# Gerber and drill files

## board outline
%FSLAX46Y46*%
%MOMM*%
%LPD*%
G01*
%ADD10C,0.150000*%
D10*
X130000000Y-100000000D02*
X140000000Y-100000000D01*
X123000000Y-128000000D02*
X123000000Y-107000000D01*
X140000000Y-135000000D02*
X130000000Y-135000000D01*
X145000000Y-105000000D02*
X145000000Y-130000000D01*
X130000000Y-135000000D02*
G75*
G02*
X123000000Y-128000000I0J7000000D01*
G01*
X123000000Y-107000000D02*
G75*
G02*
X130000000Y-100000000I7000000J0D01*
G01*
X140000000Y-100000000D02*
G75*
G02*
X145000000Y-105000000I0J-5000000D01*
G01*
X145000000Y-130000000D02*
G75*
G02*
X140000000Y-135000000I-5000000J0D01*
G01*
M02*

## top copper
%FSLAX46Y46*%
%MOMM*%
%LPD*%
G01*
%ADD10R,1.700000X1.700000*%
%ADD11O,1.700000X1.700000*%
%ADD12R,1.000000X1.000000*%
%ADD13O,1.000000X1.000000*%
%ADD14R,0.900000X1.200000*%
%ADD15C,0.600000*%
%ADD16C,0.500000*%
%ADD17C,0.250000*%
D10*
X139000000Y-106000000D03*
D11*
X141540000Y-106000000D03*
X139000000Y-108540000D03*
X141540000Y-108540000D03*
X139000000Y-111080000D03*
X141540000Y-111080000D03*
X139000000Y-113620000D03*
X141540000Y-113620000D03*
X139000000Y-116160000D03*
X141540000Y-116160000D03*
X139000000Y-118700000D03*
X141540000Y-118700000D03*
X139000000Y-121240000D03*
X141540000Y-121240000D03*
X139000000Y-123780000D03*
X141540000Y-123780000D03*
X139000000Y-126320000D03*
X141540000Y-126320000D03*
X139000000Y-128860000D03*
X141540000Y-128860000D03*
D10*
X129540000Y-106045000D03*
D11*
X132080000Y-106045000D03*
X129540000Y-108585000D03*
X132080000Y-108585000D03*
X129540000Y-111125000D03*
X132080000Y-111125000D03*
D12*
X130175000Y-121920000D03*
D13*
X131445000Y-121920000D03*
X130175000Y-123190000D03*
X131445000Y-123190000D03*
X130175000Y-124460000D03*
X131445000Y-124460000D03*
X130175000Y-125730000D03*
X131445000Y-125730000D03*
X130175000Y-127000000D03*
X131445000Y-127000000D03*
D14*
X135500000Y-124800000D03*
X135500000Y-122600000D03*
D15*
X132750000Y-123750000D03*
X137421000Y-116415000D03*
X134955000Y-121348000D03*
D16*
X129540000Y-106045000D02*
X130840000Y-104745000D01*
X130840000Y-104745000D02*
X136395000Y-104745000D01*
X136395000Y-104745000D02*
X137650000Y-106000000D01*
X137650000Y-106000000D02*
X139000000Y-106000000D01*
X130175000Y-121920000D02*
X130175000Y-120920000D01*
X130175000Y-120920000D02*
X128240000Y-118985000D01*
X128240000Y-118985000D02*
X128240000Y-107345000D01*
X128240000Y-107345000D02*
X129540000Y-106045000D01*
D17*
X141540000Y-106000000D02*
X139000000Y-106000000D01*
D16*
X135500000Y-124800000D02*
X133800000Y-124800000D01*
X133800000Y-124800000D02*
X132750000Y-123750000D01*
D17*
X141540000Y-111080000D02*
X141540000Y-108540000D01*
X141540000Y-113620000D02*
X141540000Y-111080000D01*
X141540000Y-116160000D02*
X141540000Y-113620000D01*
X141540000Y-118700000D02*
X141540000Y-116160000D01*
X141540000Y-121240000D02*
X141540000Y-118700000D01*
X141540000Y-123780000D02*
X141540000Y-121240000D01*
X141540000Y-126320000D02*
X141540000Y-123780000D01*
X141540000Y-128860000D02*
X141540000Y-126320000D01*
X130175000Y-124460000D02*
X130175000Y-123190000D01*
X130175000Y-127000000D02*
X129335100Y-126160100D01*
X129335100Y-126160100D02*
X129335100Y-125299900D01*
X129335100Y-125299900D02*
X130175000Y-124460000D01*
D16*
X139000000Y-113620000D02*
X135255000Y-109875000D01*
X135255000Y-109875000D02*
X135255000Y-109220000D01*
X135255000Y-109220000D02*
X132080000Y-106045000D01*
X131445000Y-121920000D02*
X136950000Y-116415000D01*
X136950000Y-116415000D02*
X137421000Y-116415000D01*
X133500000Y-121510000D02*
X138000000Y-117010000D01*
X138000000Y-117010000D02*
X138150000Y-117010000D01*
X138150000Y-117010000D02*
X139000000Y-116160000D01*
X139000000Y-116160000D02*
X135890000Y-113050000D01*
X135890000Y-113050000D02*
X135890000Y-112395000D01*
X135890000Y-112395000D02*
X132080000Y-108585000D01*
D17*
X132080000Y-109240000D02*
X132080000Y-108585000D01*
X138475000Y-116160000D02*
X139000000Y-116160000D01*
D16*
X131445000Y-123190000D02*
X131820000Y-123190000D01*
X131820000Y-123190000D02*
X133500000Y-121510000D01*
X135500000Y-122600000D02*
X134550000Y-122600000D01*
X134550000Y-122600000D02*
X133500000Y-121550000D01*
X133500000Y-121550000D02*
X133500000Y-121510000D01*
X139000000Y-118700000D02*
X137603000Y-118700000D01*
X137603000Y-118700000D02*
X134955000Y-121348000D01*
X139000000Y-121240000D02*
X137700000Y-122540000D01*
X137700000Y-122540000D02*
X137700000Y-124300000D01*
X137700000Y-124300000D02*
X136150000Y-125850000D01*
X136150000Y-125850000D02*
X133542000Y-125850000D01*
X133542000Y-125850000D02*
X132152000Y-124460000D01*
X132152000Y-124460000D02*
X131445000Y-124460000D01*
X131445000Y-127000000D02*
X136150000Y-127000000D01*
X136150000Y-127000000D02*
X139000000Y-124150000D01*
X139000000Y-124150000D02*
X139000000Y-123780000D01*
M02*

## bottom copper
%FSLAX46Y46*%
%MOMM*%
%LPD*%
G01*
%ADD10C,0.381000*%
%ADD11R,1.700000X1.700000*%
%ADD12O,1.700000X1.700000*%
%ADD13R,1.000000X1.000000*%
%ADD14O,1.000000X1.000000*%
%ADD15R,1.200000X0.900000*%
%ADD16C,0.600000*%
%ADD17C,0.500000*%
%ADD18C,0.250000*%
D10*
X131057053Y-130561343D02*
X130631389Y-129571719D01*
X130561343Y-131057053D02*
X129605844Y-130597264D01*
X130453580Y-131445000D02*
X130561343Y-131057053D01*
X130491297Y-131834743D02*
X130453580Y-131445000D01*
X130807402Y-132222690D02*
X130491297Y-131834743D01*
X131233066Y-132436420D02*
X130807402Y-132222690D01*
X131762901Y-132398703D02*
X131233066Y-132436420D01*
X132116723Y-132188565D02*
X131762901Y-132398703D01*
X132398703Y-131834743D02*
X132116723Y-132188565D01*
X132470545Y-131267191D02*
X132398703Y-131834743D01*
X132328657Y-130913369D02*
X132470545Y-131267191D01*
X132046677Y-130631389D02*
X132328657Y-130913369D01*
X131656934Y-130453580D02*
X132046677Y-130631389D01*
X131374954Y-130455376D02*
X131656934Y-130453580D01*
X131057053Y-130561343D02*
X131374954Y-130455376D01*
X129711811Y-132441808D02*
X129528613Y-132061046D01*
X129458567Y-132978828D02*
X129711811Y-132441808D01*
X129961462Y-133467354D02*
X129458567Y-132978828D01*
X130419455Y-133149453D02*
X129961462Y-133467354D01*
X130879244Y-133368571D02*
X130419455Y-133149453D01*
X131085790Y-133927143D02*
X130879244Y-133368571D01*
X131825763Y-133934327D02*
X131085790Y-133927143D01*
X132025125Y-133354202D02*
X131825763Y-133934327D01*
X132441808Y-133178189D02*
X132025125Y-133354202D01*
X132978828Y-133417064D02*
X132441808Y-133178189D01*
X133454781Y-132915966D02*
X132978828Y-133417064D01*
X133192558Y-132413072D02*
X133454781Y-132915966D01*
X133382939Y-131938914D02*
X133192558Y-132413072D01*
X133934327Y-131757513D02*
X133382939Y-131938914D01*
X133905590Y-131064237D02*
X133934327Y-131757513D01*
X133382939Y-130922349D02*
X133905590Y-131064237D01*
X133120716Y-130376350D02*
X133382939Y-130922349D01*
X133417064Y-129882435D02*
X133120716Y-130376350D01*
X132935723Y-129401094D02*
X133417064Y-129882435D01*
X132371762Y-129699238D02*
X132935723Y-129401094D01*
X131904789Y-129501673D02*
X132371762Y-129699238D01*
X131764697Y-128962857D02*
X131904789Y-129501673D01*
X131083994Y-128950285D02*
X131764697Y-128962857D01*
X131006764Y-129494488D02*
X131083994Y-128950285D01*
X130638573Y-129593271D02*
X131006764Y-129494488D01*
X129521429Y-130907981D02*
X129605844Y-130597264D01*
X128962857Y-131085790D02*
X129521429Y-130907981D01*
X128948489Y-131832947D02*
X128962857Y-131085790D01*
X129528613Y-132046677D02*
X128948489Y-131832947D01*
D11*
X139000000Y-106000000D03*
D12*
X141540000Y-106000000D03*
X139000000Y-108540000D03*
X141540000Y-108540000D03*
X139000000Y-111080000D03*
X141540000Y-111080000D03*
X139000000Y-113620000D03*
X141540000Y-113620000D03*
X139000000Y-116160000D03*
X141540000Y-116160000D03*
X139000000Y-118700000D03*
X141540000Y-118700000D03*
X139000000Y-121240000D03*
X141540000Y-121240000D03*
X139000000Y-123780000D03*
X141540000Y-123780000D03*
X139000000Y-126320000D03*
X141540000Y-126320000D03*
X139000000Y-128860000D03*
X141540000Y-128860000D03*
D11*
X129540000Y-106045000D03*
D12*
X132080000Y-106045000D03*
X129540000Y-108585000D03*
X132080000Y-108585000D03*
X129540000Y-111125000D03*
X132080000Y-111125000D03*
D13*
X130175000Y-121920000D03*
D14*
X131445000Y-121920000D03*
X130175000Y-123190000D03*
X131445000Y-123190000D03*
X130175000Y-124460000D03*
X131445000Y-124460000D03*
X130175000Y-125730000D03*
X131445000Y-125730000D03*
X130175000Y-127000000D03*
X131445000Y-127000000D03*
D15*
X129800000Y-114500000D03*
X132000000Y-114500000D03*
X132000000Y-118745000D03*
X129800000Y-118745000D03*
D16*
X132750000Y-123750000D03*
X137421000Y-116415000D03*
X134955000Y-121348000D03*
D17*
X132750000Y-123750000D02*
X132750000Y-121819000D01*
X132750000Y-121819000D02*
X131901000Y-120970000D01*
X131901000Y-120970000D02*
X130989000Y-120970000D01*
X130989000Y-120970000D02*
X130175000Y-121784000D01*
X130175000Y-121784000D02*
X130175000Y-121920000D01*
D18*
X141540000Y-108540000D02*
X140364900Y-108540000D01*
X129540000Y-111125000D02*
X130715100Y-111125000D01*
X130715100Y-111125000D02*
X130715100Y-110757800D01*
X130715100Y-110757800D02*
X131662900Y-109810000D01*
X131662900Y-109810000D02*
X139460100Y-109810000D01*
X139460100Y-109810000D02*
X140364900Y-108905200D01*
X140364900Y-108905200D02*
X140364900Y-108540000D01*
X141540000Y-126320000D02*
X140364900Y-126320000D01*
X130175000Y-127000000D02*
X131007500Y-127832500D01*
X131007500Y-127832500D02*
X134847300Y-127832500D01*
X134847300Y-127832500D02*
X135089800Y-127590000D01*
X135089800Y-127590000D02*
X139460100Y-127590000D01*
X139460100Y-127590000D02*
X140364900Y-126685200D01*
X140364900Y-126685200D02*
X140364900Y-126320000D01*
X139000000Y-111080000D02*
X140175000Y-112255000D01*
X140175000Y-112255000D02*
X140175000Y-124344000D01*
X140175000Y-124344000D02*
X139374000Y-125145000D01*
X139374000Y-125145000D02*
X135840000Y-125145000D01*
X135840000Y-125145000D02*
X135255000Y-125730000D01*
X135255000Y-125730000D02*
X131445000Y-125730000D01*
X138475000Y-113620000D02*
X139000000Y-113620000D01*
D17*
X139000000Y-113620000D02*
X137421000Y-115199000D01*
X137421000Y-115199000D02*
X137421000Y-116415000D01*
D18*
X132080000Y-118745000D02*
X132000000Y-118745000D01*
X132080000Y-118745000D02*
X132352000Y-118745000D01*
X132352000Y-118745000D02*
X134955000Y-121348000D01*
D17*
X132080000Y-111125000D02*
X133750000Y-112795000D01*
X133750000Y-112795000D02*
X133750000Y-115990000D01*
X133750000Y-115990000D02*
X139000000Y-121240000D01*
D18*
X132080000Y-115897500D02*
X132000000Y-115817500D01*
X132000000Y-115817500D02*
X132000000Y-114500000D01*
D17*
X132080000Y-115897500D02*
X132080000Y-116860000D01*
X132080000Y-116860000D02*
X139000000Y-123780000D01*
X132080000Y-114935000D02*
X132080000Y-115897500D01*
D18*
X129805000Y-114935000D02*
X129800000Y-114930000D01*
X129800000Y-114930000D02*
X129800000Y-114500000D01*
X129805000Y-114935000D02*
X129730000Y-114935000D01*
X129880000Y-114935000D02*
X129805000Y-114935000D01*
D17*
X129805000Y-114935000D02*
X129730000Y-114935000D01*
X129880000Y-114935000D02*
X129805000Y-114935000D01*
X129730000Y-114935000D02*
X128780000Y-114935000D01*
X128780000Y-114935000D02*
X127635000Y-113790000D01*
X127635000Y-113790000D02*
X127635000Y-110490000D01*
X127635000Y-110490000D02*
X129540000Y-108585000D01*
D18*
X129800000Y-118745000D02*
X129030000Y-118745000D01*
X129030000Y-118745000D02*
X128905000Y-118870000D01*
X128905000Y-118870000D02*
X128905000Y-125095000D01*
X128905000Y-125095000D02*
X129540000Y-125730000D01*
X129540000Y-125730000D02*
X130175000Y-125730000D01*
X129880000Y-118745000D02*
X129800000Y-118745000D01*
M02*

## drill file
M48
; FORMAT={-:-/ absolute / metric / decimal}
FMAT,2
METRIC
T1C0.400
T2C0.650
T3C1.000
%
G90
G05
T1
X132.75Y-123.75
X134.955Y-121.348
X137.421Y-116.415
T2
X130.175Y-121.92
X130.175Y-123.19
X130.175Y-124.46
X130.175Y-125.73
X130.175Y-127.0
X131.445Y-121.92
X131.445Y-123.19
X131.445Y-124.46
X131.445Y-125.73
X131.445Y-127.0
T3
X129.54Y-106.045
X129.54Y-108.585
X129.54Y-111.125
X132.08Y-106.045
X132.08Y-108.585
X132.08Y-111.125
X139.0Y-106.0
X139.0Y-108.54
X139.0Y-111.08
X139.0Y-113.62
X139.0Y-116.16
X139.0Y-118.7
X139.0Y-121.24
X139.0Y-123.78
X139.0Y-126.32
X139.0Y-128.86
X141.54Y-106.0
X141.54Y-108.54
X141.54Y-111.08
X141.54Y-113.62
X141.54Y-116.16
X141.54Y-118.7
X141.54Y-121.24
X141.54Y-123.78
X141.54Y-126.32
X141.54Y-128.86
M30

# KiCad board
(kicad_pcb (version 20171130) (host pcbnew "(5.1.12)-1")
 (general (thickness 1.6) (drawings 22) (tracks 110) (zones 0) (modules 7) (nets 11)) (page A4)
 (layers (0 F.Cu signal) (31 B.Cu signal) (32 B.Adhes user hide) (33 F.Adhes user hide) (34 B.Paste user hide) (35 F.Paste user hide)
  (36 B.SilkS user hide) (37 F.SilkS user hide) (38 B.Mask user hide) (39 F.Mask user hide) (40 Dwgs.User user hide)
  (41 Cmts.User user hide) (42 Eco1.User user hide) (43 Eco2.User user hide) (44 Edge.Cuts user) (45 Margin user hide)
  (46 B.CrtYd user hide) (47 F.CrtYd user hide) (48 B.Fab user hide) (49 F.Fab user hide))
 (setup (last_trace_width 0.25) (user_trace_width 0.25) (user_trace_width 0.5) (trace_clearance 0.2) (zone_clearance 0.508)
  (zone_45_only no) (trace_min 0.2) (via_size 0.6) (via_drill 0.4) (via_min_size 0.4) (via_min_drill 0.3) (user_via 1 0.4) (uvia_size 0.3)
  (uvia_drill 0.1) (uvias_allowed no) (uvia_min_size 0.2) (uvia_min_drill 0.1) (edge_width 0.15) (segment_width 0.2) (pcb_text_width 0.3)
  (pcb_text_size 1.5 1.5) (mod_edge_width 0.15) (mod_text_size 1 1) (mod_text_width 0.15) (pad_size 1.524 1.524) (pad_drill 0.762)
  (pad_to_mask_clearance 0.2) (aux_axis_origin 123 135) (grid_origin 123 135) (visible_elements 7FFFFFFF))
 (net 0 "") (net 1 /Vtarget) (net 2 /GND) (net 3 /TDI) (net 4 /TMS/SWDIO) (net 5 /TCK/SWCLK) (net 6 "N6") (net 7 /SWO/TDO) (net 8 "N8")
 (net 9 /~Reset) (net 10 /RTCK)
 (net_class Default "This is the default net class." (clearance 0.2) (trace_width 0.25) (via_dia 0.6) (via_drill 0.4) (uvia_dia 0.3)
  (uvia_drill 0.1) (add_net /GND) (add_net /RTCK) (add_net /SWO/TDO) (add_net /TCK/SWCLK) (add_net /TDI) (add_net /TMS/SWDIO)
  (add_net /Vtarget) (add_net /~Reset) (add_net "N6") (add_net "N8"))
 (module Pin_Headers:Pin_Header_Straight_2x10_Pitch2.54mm (layer F.Cu) (at 139 106)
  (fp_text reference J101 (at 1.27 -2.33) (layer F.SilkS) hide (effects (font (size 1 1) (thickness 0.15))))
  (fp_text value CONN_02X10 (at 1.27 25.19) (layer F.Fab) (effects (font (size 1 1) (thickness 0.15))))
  (pad 1 thru_hole rect (at 0 0) (size 1.7 1.7) (drill 1) (layers *.Cu *.Mask) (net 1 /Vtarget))
  (pad 2 thru_hole oval (at 2.54 0) (size 1.7 1.7) (drill 1) (layers *.Cu *.Mask) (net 1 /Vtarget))
  (pad 3 thru_hole oval (at 0 2.54) (size 1.7 1.7) (drill 1) (layers *.Cu *.Mask))
  (pad 4 thru_hole oval (at 2.54 2.54) (size 1.7 1.7) (drill 1) (layers *.Cu *.Mask) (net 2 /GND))
  (pad 5 thru_hole oval (at 0 5.08) (size 1.7 1.7) (drill 1) (layers *.Cu *.Mask) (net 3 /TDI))
  (pad 6 thru_hole oval (at 2.54 5.08) (size 1.7 1.7) (drill 1) (layers *.Cu *.Mask) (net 2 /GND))
  (pad 7 thru_hole oval (at 0 7.62) (size 1.7 1.7) (drill 1) (layers *.Cu *.Mask) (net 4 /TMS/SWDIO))
  (pad 8 thru_hole oval (at 2.54 7.62) (size 1.7 1.7) (drill 1) (layers *.Cu *.Mask) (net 2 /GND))
  (pad 9 thru_hole oval (at 0 10.16) (size 1.7 1.7) (drill 1) (layers *.Cu *.Mask) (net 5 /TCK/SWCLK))
  (pad 10 thru_hole oval (at 2.54 10.16) (size 1.7 1.7) (drill 1) (layers *.Cu *.Mask) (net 2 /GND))
  (pad 11 thru_hole oval (at 0 12.7) (size 1.7 1.7) (drill 1) (layers *.Cu *.Mask) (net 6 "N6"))
  (pad 12 thru_hole oval (at 2.54 12.7) (size 1.7 1.7) (drill 1) (layers *.Cu *.Mask) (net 2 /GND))
  (pad 13 thru_hole oval (at 0 15.24) (size 1.7 1.7) (drill 1) (layers *.Cu *.Mask) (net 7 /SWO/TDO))
  (pad 14 thru_hole oval (at 2.54 15.24) (size 1.7 1.7) (drill 1) (layers *.Cu *.Mask) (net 2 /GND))
  (pad 15 thru_hole oval (at 0 17.78) (size 1.7 1.7) (drill 1) (layers *.Cu *.Mask) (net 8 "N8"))
  (pad 16 thru_hole oval (at 2.54 17.78) (size 1.7 1.7) (drill 1) (layers *.Cu *.Mask) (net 2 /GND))
  (pad 17 thru_hole oval (at 0 20.32) (size 1.7 1.7) (drill 1) (layers *.Cu *.Mask))
  (pad 18 thru_hole oval (at 2.54 20.32) (size 1.7 1.7) (drill 1) (layers *.Cu *.Mask) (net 2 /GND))
  (pad 19 thru_hole oval (at 0 22.86) (size 1.7 1.7) (drill 1) (layers *.Cu *.Mask))
  (pad 20 thru_hole oval (at 2.54 22.86) (size 1.7 1.7) (drill 1) (layers *.Cu *.Mask) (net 2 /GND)))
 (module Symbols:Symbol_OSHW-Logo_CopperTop (layer B.Cu) (at 131.445 131.445 45)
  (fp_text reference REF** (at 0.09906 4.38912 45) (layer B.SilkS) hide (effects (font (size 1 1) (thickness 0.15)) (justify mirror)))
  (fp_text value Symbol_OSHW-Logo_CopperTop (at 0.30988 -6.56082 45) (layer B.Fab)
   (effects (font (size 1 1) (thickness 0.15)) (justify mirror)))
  (fp_line (start 0.35052 -0.89916) (end 0.7493 -1.89992) (layer B.Cu) (width 0.381))
  (fp_line (start -0.35052 -0.89916) (end -0.70104 -1.89992) (layer B.Cu) (width 0.381))
  (fp_line (start -0.70104 -0.70104) (end -0.35052 -0.89916) (layer B.Cu) (width 0.381))
  (fp_line (start -0.94996 -0.39878) (end -0.70104 -0.70104) (layer B.Cu) (width 0.381))
  (fp_line (start -1.00076 0.09906) (end -0.94996 -0.39878) (layer B.Cu) (width 0.381))
  (fp_line (start -0.8509 0.55118) (end -1.00076 0.09906) (layer B.Cu) (width 0.381))
  (fp_line (start -0.44958 0.89916) (end -0.8509 0.55118) (layer B.Cu) (width 0.381))
  (fp_line (start -0.0508 1.00076) (end -0.44958 0.89916) (layer B.Cu) (width 0.381))
  (fp_line (start 0.39878 0.94996) (end -0.0508 1.00076) (layer B.Cu) (width 0.381))
  (fp_line (start 0.8509 0.59944) (end 0.39878 0.94996) (layer B.Cu) (width 0.381))
  (fp_line (start 1.00076 0.24892) (end 0.8509 0.59944) (layer B.Cu) (width 0.381))
  (fp_line (start 1.00076 -0.14986) (end 1.00076 0.24892) (layer B.Cu) (width 0.381))
  (fp_line (start 0.8509 -0.55118) (end 1.00076 -0.14986) (layer B.Cu) (width 0.381))
  (fp_line (start 0.65024 -0.7493) (end 0.8509 -0.55118) (layer B.Cu) (width 0.381))
  (fp_line (start 0.35052 -0.89916) (end 0.65024 -0.7493) (layer B.Cu) (width 0.381))
  (fp_line (start -1.9304 -0.5207) (end -1.7907 -0.91948) (layer B.Cu) (width 0.381))
  (fp_line (start -2.4892 -0.32004) (end -1.9304 -0.5207) (layer B.Cu) (width 0.381))
  (fp_line (start -2.47904 0.381) (end -2.4892 -0.32004) (layer B.Cu) (width 0.381))
  (fp_line (start -1.9304 0.48006) (end -2.47904 0.381) (layer B.Cu) (width 0.381))
  (fp_line (start -1.76022 0.96012) (end -1.9304 0.48006) (layer B.Cu) (width 0.381))
  (fp_line (start -2.00914 1.50114) (end -1.76022 0.96012) (layer B.Cu) (width 0.381))
  (fp_line (start -1.49098 2.02946) (end -2.00914 1.50114) (layer B.Cu) (width 0.381))
  (fp_line (start -0.9398 1.76022) (end -1.49098 2.02946) (layer B.Cu) (width 0.381))
  (fp_line (start -0.5207 1.9304) (end -0.9398 1.76022) (layer B.Cu) (width 0.381))
  (fp_line (start -0.30988 2.47904) (end -0.5207 1.9304) (layer B.Cu) (width 0.381))
  (fp_line (start 0.381 2.46126) (end -0.30988 2.47904) (layer B.Cu) (width 0.381))
  (fp_line (start 0.55118 1.92024) (end 0.381 2.46126) (layer B.Cu) (width 0.381))
  (fp_line (start 1.02108 1.71958) (end 0.55118 1.92024) (layer B.Cu) (width 0.381))
  (fp_line (start 1.53924 1.9812) (end 1.02108 1.71958) (layer B.Cu) (width 0.381))
  (fp_line (start 2.00914 1.47066) (end 1.53924 1.9812) (layer B.Cu) (width 0.381))
  (fp_line (start 1.7399 1.00076) (end 2.00914 1.47066) (layer B.Cu) (width 0.381))
  (fp_line (start 1.94056 0.42926) (end 1.7399 1.00076) (layer B.Cu) (width 0.381))
  (fp_line (start 2.49936 0.28956) (end 1.94056 0.42926) (layer B.Cu) (width 0.381))
  (fp_line (start 2.49936 -0.39116) (end 2.49936 0.28956) (layer B.Cu) (width 0.381))
  (fp_line (start 1.88976 -0.57912) (end 2.49936 -0.39116) (layer B.Cu) (width 0.381))
  (fp_line (start 1.69926 -1.04902) (end 1.88976 -0.57912) (layer B.Cu) (width 0.381))
  (fp_line (start 1.9812 -1.52908) (end 1.69926 -1.04902) (layer B.Cu) (width 0.381))
  (fp_line (start 1.50876 -2.0193) (end 1.9812 -1.52908) (layer B.Cu) (width 0.381))
  (fp_line (start 1.06934 -1.6891) (end 1.50876 -2.0193) (layer B.Cu) (width 0.381))
  (fp_line (start 0.73914 -1.8796) (end 1.06934 -1.6891) (layer B.Cu) (width 0.381))
  (fp_line (start -0.98044 -1.7399) (end -0.70104 -1.89992) (layer B.Cu) (width 0.381))
  (fp_line (start -1.50114 -2.00914) (end -0.98044 -1.7399) (layer B.Cu) (width 0.381))
  (fp_line (start -2.03962 -1.49098) (end -1.50114 -2.00914) (layer B.Cu) (width 0.381))
  (fp_line (start -1.78054 -0.92964) (end -2.03962 -1.49098) (layer B.Cu) (width 0.381)))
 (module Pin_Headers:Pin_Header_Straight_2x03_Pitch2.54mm (layer F.Cu) (at 129.54 106.045)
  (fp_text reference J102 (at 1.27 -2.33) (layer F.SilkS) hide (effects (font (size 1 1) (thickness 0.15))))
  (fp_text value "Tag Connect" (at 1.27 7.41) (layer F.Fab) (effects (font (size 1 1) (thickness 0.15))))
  (pad 1 thru_hole rect (at 0 0) (size 1.7 1.7) (drill 1) (layers *.Cu *.Mask) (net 1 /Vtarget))
  (pad 2 thru_hole oval (at 2.54 0) (size 1.7 1.7) (drill 1) (layers *.Cu *.Mask) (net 4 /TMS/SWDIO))
  (pad 3 thru_hole oval (at 0 2.54) (size 1.7 1.7) (drill 1) (layers *.Cu *.Mask) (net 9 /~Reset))
  (pad 4 thru_hole oval (at 2.54 2.54) (size 1.7 1.7) (drill 1) (layers *.Cu *.Mask) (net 5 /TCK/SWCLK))
  (pad 5 thru_hole oval (at 0 5.08) (size 1.7 1.7) (drill 1) (layers *.Cu *.Mask) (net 2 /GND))
  (pad 6 thru_hole oval (at 2.54 5.08) (size 1.7 1.7) (drill 1) (layers *.Cu *.Mask) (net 7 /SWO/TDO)))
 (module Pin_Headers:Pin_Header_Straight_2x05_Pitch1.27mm (layer F.Cu) (at 130.175 121.92)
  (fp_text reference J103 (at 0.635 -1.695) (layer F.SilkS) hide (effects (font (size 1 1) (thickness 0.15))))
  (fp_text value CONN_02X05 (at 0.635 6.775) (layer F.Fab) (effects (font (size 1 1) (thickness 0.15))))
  (pad 1 thru_hole rect (at 0 0) (size 1 1) (drill 0.65) (layers *.Cu *.Mask) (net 1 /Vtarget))
  (pad 2 thru_hole oval (at 1.27 0) (size 1 1) (drill 0.65) (layers *.Cu *.Mask) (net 4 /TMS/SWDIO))
  (pad 3 thru_hole oval (at 0 1.27) (size 1 1) (drill 0.65) (layers *.Cu *.Mask) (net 2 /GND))
  (pad 4 thru_hole oval (at 1.27 1.27) (size 1 1) (drill 0.65) (layers *.Cu *.Mask) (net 5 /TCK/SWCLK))
  (pad 5 thru_hole oval (at 0 2.54) (size 1 1) (drill 0.65) (layers *.Cu *.Mask) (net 2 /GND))
  (pad 6 thru_hole oval (at 1.27 2.54) (size 1 1) (drill 0.65) (layers *.Cu *.Mask) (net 7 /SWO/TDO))
  (pad 7 thru_hole oval (at 0 3.81) (size 1 1) (drill 0.65) (layers *.Cu *.Mask) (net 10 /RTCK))
  (pad 8 thru_hole oval (at 1.27 3.81) (size 1 1) (drill 0.65) (layers *.Cu *.Mask) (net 3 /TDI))
  (pad 9 thru_hole oval (at 0 5.08) (size 1 1) (drill 0.65) (layers *.Cu *.Mask) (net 2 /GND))
  (pad 10 thru_hole oval (at 1.27 5.08) (size 1 1) (drill 0.65) (layers *.Cu *.Mask) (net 8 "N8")))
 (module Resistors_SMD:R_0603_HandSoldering (layer B.Cu) (at 130.9 114.5)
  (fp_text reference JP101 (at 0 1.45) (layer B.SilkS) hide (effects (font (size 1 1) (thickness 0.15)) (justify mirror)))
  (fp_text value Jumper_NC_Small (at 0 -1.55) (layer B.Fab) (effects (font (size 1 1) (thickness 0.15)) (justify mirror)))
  (pad 1 smd rect (at -1.1 0) (size 1.2 0.9) (layers B.Cu B.Paste B.Mask) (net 9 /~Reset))
  (pad 2 smd rect (at 1.1 0) (size 1.2 0.9) (layers B.Cu B.Paste B.Mask) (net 8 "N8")))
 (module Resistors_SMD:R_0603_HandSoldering (layer B.Cu) (at 130.9 118.745 180)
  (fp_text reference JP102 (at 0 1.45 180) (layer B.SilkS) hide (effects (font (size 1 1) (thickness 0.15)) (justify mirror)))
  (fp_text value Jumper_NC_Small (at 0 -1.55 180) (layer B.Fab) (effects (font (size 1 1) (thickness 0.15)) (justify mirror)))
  (pad 1 smd rect (at -1.1 0 180) (size 1.2 0.9) (layers B.Cu B.Paste B.Mask) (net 6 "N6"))
  (pad 2 smd rect (at 1.1 0 180) (size 1.2 0.9) (layers B.Cu B.Paste B.Mask) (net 10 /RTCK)))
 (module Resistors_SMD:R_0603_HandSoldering (layer F.Cu) (at 135.5 123.7 90)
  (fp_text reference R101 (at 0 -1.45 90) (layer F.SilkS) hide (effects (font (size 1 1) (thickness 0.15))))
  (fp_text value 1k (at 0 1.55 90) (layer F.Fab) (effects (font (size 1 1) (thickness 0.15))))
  (pad 1 smd rect (at -1.1 0 90) (size 1.2 0.9) (layers F.Cu F.Paste F.Mask) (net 1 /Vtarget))
  (pad 2 smd rect (at 1.1 0 90) (size 1.2 0.9) (layers F.Cu F.Paste F.Mask) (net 5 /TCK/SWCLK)))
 (gr_line (start 130 100) (end 140 100) (layer Edge.Cuts) (width 0.15))
 (gr_line (start 123 128) (end 123 107) (layer Edge.Cuts) (width 0.15))
 (gr_line (start 140 135) (end 130 135) (layer Edge.Cuts) (width 0.15))
 (gr_line (start 145 105) (end 145 130) (layer Edge.Cuts) (width 0.15))
 (gr_arc (start 130 128) (end 130 135) (angle 90) (layer Edge.Cuts) (width 0.15))
 (gr_arc (start 130 107) (end 123 107) (angle 90) (layer Edge.Cuts) (width 0.15))
 (gr_arc (start 140 105) (end 140 100) (angle 90) (layer Edge.Cuts) (width 0.15))
 (gr_arc (start 140 130) (end 145 130) (angle 90) (layer Edge.Cuts) (width 0.15))
 (segment (start 129.54 106.045) (end 130.84 104.745) (width 0.5) (layer F.Cu) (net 1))
 (segment (start 130.84 104.745) (end 136.395 104.745) (width 0.5) (layer F.Cu) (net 1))
 (segment (start 136.395 104.745) (end 137.65 106) (width 0.5) (layer F.Cu) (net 1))
 (segment (start 137.65 106) (end 139 106) (width 0.5) (layer F.Cu) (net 1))
 (segment (start 130.175 121.92) (end 130.175 120.92) (width 0.5) (layer F.Cu) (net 1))
 (segment (start 130.175 120.92) (end 128.24 118.985) (width 0.5) (layer F.Cu) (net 1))
 (segment (start 128.24 118.985) (end 128.24 107.345) (width 0.5) (layer F.Cu) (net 1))
 (segment (start 128.24 107.345) (end 129.54 106.045) (width 0.5) (layer F.Cu) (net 1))
 (segment (start 141.54 106) (end 139 106) (width 0.25) (layer F.Cu) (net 1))
 (segment (start 135.5 124.8) (end 133.8 124.8) (width 0.5) (layer F.Cu) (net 1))
 (segment (start 133.8 124.8) (end 132.75 123.75) (width 0.5) (layer F.Cu) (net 1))
 (segment (start 132.75 123.75) (end 132.75 121.819) (width 0.5) (layer B.Cu) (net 1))
 (segment (start 132.75 121.819) (end 131.901 120.97) (width 0.5) (layer B.Cu) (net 1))
 (segment (start 131.901 120.97) (end 130.989 120.97) (width 0.5) (layer B.Cu) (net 1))
 (segment (start 130.989 120.97) (end 130.175 121.784) (width 0.5) (layer B.Cu) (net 1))
 (segment (start 130.175 121.784) (end 130.175 121.92) (width 0.5) (layer B.Cu) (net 1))
 (via (at 132.75 123.75) (size 0.6) (layers F.Cu B.Cu) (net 1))
 (segment (start 141.54 111.08) (end 141.54 108.54) (width 0.25) (layer F.Cu) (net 2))
 (segment (start 141.54 113.62) (end 141.54 111.08) (width 0.25) (layer F.Cu) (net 2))
 (segment (start 141.54 116.16) (end 141.54 113.62) (width 0.25) (layer F.Cu) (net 2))
 (segment (start 141.54 118.7) (end 141.54 116.16) (width 0.25) (layer F.Cu) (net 2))
 (segment (start 141.54 121.24) (end 141.54 118.7) (width 0.25) (layer F.Cu) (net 2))
 (segment (start 141.54 123.78) (end 141.54 121.24) (width 0.25) (layer F.Cu) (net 2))
 (segment (start 141.54 126.32) (end 141.54 123.78) (width 0.25) (layer F.Cu) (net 2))
 (segment (start 141.54 128.86) (end 141.54 126.32) (width 0.25) (layer F.Cu) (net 2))
 (segment (start 141.54 108.54) (end 140.3649 108.54) (width 0.25) (layer B.Cu) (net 2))
 (segment (start 129.54 111.125) (end 130.7151 111.125) (width 0.25) (layer B.Cu) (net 2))
 (segment (start 130.7151 111.125) (end 130.7151 110.7578) (width 0.25) (layer B.Cu) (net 2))
 (segment (start 130.7151 110.7578) (end 131.6629 109.81) (width 0.25) (layer B.Cu) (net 2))
 (segment (start 131.6629 109.81) (end 139.4601 109.81) (width 0.25) (layer B.Cu) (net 2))
 (segment (start 139.4601 109.81) (end 140.3649 108.9052) (width 0.25) (layer B.Cu) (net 2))
 (segment (start 140.3649 108.9052) (end 140.3649 108.54) (width 0.25) (layer B.Cu) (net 2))
 (segment (start 141.54 126.32) (end 140.3649 126.32) (width 0.25) (layer B.Cu) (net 2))
 (segment (start 130.175 127) (end 131.0075 127.8325) (width 0.25) (layer B.Cu) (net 2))
 (segment (start 131.0075 127.8325) (end 134.8473 127.8325) (width 0.25) (layer B.Cu) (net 2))
 (segment (start 134.8473 127.8325) (end 135.0898 127.59) (width 0.25) (layer B.Cu) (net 2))
 (segment (start 135.0898 127.59) (end 139.4601 127.59) (width 0.25) (layer B.Cu) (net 2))
 (segment (start 139.4601 127.59) (end 140.3649 126.6852) (width 0.25) (layer B.Cu) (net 2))
 (segment (start 140.3649 126.6852) (end 140.3649 126.32) (width 0.25) (layer B.Cu) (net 2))
 (segment (start 130.175 124.46) (end 130.175 123.19) (width 0.25) (layer F.Cu) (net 2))
 (segment (start 130.175 127) (end 129.3351 126.1601) (width 0.25) (layer F.Cu) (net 2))
 (segment (start 129.3351 126.1601) (end 129.3351 125.2999) (width 0.25) (layer F.Cu) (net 2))
 (segment (start 129.3351 125.2999) (end 130.175 124.46) (width 0.25) (layer F.Cu) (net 2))
 (segment (start 139 111.08) (end 140.175 112.255) (width 0.25) (layer B.Cu) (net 3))
 (segment (start 140.175 112.255) (end 140.175 124.344) (width 0.25) (layer B.Cu) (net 3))
 (segment (start 140.175 124.344) (end 139.374 125.145) (width 0.25) (layer B.Cu) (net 3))
 (segment (start 139.374 125.145) (end 135.84 125.145) (width 0.25) (layer B.Cu) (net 3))
 (segment (start 135.84 125.145) (end 135.255 125.73) (width 0.25) (layer B.Cu) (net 3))
 (segment (start 135.255 125.73) (end 131.445 125.73) (width 0.25) (layer B.Cu) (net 3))
 (segment (start 138.475 113.62) (end 139 113.62) (width 0.25) (layer B.Cu) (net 4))
 (segment (start 139 113.62) (end 135.255 109.875) (width 0.5) (layer F.Cu) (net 4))
 (segment (start 135.255 109.875) (end 135.255 109.22) (width 0.5) (layer F.Cu) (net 4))
 (segment (start 135.255 109.22) (end 132.08 106.045) (width 0.5) (layer F.Cu) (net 4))
 (segment (start 131.445 121.92) (end 136.95 116.415) (width 0.5) (layer F.Cu) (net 4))
 (segment (start 136.95 116.415) (end 137.421 116.415) (width 0.5) (layer F.Cu) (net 4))
 (segment (start 139 113.62) (end 137.421 115.199) (width 0.5) (layer B.Cu) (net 4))
 (segment (start 137.421 115.199) (end 137.421 116.415) (width 0.5) (layer B.Cu) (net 4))
 (via (at 137.421 116.415) (size 0.6) (layers F.Cu B.Cu) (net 4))
 (segment (start 133.5 121.51) (end 138 117.01) (width 0.5) (layer F.Cu) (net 5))
 (segment (start 138 117.01) (end 138.15 117.01) (width 0.5) (layer F.Cu) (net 5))
 (segment (start 138.15 117.01) (end 139 116.16) (width 0.5) (layer F.Cu) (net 5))
 (segment (start 139 116.16) (end 135.89 113.05) (width 0.5) (layer F.Cu) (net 5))
 (segment (start 135.89 113.05) (end 135.89 112.395) (width 0.5) (layer F.Cu) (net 5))
 (segment (start 135.89 112.395) (end 132.08 108.585) (width 0.5) (layer F.Cu) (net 5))
 (segment (start 132.08 109.24) (end 132.08 108.585) (width 0.25) (layer F.Cu) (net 5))
 (segment (start 138.475 116.16) (end 139 116.16) (width 0.25) (layer F.Cu) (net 5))
 (segment (start 131.445 123.19) (end 131.82 123.19) (width 0.5) (layer F.Cu) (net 5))
 (segment (start 131.82 123.19) (end 133.5 121.51) (width 0.5) (layer F.Cu) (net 5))
 (segment (start 135.5 122.6) (end 134.55 122.6) (width 0.5) (layer F.Cu) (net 5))
 (segment (start 134.55 122.6) (end 133.5 121.55) (width 0.5) (layer F.Cu) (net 5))
 (segment (start 133.5 121.55) (end 133.5 121.51) (width 0.5) (layer F.Cu) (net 5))
 (segment (start 132.08 118.745) (end 132 118.745) (width 0.25) (layer B.Cu) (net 6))
 (segment (start 132.08 118.745) (end 132.352 118.745) (width 0.25) (layer B.Cu) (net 6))
 (segment (start 132.352 118.745) (end 134.955 121.348) (width 0.25) (layer B.Cu) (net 6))
 (segment (start 139 118.7) (end 137.603 118.7) (width 0.5) (layer F.Cu) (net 6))
 (segment (start 137.603 118.7) (end 134.955 121.348) (width 0.5) (layer F.Cu) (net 6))
 (via (at 134.955 121.348) (size 0.6) (layers F.Cu B.Cu) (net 6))
 (segment (start 139 121.24) (end 137.7 122.54) (width 0.5) (layer F.Cu) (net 7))
 (segment (start 137.7 122.54) (end 137.7 124.3) (width 0.5) (layer F.Cu) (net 7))
 (segment (start 137.7 124.3) (end 136.15 125.85) (width 0.5) (layer F.Cu) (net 7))
 (segment (start 136.15 125.85) (end 133.542 125.85) (width 0.5) (layer F.Cu) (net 7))
 (segment (start 133.542 125.85) (end 132.152 124.46) (width 0.5) (layer F.Cu) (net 7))
 (segment (start 132.152 124.46) (end 131.445 124.46) (width 0.5) (layer F.Cu) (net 7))
 (segment (start 132.08 111.125) (end 133.75 112.795) (width 0.5) (layer B.Cu) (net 7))
 (segment (start 133.75 112.795) (end 133.75 115.99) (width 0.5) (layer B.Cu) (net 7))
 (segment (start 133.75 115.99) (end 139 121.24) (width 0.5) (layer B.Cu) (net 7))
 (segment (start 132.08 115.8975) (end 132 115.8175) (width 0.25) (layer B.Cu) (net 8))
 (segment (start 132 115.8175) (end 132 114.5) (width 0.25) (layer B.Cu) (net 8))
 (segment (start 132.08 115.8975) (end 132.08 116.86) (width 0.5) (layer B.Cu) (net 8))
 (segment (start 132.08 116.86) (end 139 123.78) (width 0.5) (layer B.Cu) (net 8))
 (segment (start 132.08 114.935) (end 132.08 115.8975) (width 0.5) (layer B.Cu) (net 8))
 (segment (start 131.445 127) (end 136.15 127) (width 0.5) (layer F.Cu) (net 8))
 (segment (start 136.15 127) (end 139 124.15) (width 0.5) (layer F.Cu) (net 8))
 (segment (start 139 124.15) (end 139 123.78) (width 0.5) (layer F.Cu) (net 8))
 (segment (start 129.805 114.935) (end 129.8 114.93) (width 0.25) (layer B.Cu) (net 9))
 (segment (start 129.8 114.93) (end 129.8 114.5) (width 0.25) (layer B.Cu) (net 9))
 (segment (start 129.805 114.935) (end 129.73 114.935) (width 0.25) (layer B.Cu) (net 9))
 (segment (start 129.88 114.935) (end 129.805 114.935) (width 0.25) (layer B.Cu) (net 9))
 (segment (start 129.805 114.935) (end 129.73 114.935) (width 0.5) (layer B.Cu) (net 9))
 (segment (start 129.88 114.935) (end 129.805 114.935) (width 0.5) (layer B.Cu) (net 9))
 (segment (start 129.73 114.935) (end 128.78 114.935) (width 0.5) (layer B.Cu) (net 9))
 (segment (start 128.78 114.935) (end 127.635 113.79) (width 0.5) (layer B.Cu) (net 9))
 (segment (start 127.635 113.79) (end 127.635 110.49) (width 0.5) (layer B.Cu) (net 9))
 (segment (start 127.635 110.49) (end 129.54 108.585) (width 0.5) (layer B.Cu) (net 9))
 (segment (start 129.8 118.745) (end 129.03 118.745) (width 0.25) (layer B.Cu) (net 10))
 (segment (start 129.03 118.745) (end 128.905 118.87) (width 0.25) (layer B.Cu) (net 10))
 (segment (start 128.905 118.87) (end 128.905 125.095) (width 0.25) (layer B.Cu) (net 10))
 (segment (start 128.905 125.095) (end 129.54 125.73) (width 0.25) (layer B.Cu) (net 10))
 (segment (start 129.54 125.73) (end 130.175 125.73) (width 0.25) (layer B.Cu) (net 10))
 (segment (start 129.88 118.745) (end 129.8 118.745) (width 0.25) (layer B.Cu) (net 10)))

